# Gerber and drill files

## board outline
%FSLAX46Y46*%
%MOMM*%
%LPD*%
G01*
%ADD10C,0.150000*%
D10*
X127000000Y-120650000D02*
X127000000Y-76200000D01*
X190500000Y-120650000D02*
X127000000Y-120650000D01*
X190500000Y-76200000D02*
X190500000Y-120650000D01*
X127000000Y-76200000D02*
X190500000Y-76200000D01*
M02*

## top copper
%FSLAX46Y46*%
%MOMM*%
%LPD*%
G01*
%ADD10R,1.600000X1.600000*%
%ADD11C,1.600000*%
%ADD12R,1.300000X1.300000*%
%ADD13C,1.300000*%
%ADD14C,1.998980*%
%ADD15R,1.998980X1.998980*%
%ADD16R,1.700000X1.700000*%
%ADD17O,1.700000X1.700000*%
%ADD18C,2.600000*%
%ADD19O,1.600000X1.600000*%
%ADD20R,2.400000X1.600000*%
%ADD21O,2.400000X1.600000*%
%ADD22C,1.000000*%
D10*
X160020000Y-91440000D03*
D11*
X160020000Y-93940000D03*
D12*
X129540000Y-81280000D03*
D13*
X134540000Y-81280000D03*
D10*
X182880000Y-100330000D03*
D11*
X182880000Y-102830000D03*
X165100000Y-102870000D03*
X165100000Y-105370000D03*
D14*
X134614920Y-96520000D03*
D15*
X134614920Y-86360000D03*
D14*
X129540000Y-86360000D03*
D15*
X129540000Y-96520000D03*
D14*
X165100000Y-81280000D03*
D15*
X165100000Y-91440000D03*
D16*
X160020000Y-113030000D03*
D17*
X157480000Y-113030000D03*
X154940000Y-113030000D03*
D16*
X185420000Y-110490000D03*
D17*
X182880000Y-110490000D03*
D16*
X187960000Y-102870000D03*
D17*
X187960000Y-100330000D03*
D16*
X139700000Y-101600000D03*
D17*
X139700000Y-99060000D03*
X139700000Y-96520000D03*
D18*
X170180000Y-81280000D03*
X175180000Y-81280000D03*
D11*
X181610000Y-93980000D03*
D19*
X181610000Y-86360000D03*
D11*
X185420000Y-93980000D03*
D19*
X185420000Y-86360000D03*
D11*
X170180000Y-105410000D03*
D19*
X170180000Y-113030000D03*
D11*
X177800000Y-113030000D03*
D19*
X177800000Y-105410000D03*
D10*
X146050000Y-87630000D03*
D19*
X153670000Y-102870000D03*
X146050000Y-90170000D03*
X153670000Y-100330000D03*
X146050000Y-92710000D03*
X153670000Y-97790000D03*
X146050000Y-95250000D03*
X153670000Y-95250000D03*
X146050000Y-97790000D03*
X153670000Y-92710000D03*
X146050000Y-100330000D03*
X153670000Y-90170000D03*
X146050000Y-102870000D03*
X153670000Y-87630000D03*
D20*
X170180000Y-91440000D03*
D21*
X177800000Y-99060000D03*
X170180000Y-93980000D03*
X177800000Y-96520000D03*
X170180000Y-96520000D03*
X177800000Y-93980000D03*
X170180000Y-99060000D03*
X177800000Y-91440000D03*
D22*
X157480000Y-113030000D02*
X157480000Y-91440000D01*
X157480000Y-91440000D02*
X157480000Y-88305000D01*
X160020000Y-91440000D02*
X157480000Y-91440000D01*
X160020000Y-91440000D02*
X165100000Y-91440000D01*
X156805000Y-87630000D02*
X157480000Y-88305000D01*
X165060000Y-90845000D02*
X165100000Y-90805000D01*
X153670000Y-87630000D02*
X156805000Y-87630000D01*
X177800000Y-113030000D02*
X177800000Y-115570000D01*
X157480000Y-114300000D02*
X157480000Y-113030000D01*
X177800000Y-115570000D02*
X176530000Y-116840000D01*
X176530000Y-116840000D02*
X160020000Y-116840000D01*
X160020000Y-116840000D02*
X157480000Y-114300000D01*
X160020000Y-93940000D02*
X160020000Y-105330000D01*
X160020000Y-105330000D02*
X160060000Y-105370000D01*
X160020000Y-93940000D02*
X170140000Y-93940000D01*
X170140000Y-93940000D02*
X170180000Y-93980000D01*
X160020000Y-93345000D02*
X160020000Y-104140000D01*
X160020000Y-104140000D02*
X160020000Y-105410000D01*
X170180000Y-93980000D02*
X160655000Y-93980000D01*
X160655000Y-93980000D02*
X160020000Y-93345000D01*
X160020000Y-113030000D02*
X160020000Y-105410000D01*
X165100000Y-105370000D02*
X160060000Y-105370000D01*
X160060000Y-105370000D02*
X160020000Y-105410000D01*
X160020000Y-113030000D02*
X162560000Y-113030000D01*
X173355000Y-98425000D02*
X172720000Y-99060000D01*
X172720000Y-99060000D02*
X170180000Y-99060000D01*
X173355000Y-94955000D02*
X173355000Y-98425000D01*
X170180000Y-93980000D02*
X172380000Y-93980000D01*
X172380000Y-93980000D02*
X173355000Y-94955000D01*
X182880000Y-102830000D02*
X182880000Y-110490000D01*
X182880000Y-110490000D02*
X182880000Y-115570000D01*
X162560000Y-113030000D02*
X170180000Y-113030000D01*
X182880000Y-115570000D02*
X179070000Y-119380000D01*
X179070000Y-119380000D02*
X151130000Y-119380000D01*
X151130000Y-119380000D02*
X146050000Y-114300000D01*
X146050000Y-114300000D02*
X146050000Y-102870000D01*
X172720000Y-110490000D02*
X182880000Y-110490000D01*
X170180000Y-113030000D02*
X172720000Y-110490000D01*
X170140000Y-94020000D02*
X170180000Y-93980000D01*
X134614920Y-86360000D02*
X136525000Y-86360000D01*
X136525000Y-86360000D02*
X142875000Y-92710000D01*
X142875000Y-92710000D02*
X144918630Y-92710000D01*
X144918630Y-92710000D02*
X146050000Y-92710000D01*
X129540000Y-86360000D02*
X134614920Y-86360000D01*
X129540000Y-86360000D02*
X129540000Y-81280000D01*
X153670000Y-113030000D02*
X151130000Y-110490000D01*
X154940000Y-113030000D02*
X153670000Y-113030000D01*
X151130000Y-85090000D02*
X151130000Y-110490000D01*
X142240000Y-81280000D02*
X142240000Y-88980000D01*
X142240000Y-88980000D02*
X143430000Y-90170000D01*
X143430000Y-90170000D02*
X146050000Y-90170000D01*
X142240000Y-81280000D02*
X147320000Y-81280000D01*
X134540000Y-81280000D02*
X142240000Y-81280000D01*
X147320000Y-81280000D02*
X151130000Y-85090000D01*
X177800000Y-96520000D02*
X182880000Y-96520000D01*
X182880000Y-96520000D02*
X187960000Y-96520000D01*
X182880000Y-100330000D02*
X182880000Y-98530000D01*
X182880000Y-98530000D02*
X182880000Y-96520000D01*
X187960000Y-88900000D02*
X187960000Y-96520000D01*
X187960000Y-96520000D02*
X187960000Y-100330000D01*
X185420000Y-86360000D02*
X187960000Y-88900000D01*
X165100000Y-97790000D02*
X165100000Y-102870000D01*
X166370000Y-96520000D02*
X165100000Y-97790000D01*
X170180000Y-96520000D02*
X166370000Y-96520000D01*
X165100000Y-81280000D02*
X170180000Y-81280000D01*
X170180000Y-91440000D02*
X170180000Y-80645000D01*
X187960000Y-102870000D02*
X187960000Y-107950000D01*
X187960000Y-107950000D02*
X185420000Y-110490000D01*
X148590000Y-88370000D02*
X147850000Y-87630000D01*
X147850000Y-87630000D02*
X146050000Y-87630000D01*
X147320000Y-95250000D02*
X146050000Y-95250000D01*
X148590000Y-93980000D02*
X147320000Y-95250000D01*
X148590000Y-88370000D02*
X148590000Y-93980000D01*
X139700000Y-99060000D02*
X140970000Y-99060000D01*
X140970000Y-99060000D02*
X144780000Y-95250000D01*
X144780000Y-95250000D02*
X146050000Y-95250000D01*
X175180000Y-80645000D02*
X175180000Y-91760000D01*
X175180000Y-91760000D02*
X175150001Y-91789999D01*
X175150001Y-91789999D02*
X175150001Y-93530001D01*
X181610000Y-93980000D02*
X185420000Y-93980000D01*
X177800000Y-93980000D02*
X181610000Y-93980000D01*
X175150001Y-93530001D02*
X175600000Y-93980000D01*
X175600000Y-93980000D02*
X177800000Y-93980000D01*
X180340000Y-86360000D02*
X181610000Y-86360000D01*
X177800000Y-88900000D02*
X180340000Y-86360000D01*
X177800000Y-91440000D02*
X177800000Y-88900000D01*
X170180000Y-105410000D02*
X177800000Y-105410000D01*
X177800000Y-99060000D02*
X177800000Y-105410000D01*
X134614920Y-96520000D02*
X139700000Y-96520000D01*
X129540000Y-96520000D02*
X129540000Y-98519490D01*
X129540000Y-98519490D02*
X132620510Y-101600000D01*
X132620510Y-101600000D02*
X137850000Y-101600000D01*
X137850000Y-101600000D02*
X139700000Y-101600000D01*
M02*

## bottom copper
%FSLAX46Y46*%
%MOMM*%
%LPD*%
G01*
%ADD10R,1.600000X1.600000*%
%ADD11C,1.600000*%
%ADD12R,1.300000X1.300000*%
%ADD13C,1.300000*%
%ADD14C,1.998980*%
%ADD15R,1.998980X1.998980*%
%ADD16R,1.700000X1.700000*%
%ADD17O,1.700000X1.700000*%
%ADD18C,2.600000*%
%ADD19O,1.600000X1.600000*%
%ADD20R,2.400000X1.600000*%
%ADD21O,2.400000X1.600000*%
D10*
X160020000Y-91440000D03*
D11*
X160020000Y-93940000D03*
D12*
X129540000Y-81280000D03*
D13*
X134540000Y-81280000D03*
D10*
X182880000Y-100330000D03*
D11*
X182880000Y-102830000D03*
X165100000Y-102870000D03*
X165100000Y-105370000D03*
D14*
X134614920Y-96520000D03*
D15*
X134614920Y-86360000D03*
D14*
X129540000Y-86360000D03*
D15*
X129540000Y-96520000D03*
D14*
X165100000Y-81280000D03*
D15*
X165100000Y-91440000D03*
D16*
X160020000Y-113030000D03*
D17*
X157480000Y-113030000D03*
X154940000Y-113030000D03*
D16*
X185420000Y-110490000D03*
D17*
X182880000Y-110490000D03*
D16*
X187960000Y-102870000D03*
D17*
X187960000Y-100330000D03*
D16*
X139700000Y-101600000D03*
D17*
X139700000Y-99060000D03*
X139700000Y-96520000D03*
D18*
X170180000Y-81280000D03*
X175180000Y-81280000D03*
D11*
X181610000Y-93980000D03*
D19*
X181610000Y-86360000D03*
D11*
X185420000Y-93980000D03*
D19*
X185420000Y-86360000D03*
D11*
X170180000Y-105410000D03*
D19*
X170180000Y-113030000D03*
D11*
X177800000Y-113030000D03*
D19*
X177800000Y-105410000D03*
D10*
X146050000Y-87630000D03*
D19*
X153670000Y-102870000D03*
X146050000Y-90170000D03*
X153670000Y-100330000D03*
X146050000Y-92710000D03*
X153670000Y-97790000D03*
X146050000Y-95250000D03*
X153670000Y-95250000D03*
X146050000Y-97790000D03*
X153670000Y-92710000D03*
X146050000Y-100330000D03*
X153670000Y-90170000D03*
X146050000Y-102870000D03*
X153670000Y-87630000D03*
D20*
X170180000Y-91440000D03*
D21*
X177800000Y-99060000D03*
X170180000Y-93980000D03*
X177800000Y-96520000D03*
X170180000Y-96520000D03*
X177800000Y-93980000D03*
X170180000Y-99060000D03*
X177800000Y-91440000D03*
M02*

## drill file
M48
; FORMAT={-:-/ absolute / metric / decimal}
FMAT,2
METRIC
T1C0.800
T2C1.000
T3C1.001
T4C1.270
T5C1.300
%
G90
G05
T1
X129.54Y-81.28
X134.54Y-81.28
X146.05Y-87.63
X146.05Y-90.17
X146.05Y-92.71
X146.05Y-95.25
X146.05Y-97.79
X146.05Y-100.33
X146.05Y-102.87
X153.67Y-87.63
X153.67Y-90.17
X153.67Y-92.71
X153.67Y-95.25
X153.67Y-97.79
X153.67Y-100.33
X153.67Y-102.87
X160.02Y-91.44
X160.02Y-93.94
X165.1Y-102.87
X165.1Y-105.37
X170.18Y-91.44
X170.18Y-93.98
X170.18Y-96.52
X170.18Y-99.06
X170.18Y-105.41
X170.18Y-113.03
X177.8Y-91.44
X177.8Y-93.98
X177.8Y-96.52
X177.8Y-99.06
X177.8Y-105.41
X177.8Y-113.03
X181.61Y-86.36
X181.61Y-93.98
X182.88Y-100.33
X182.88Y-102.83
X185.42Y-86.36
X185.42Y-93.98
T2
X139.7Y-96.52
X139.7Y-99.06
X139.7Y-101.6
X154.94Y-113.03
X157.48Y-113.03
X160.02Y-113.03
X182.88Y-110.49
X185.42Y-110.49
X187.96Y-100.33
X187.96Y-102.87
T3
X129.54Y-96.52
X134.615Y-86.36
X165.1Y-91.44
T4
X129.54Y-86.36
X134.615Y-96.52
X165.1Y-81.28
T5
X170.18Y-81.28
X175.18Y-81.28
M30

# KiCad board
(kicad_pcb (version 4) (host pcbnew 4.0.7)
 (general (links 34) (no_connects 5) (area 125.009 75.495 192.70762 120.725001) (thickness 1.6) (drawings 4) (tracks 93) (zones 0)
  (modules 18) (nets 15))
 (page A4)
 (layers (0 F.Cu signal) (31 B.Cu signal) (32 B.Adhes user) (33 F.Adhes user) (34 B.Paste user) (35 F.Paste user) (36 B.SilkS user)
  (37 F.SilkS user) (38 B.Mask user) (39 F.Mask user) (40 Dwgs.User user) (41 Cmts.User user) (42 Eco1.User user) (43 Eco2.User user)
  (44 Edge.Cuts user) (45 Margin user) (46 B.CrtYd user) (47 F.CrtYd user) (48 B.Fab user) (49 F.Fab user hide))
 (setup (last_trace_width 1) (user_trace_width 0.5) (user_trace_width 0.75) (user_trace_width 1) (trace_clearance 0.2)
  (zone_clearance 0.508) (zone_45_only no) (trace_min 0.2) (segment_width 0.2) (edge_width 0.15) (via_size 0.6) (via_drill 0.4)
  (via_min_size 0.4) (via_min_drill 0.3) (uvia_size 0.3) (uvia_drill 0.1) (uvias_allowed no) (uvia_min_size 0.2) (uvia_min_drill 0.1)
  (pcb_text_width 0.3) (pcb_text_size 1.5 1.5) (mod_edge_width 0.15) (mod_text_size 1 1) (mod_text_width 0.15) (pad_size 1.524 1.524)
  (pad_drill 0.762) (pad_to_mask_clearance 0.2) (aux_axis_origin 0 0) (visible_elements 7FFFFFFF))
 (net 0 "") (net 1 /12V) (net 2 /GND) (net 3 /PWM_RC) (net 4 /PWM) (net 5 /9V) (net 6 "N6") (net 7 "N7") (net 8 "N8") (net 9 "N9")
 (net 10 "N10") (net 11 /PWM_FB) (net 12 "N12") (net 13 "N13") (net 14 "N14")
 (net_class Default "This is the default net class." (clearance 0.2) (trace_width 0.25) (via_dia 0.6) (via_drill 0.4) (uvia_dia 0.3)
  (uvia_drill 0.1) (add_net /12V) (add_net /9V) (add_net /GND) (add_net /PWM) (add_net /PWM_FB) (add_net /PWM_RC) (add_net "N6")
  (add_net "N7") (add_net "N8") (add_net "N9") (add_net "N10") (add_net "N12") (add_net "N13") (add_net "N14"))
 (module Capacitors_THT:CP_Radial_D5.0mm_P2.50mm (layer F.Cu) (at 160.02 91.44 270)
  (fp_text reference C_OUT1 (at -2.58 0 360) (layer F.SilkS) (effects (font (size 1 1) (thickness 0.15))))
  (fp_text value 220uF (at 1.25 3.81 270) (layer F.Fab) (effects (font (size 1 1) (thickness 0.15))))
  (pad 1 thru_hole rect (at 0 0 270) (size 1.6 1.6) (drill 0.8) (layers *.Cu *.Mask) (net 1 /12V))
  (pad 2 thru_hole circle (at 2.5 0 270) (size 1.6 1.6) (drill 0.8) (layers *.Cu *.Mask) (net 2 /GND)))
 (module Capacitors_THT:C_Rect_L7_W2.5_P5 (layer F.Cu) (at 129.54 81.28)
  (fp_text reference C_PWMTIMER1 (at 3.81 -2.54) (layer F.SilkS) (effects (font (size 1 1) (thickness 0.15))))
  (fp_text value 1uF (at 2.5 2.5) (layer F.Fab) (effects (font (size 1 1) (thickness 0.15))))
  (pad 1 thru_hole rect (at 0 0) (size 1.3 1.3) (drill 0.8) (layers *.Cu *.Mask) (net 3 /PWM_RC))
  (pad 2 thru_hole circle (at 5 0) (size 1.3 1.3) (drill 0.8) (layers *.Cu *.Mask) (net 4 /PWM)))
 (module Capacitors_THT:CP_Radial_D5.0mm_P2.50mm (layer F.Cu) (at 182.88 100.33 270)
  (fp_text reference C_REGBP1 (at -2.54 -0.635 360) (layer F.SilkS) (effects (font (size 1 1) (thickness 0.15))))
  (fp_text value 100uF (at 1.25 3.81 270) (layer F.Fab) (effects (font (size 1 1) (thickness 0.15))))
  (pad 1 thru_hole rect (at 0 0 270) (size 1.6 1.6) (drill 0.8) (layers *.Cu *.Mask) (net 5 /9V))
  (pad 2 thru_hole circle (at 2.5 0 270) (size 1.6 1.6) (drill 0.8) (layers *.Cu *.Mask) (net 2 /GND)))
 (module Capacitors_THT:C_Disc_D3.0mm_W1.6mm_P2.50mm (layer F.Cu) (at 165.1 102.87 270)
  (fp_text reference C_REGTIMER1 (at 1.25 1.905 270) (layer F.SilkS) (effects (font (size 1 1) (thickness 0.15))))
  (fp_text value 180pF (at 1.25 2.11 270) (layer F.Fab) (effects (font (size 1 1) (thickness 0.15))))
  (pad 1 thru_hole circle (at 0 0 270) (size 1.6 1.6) (drill 0.8) (layers *.Cu *.Mask) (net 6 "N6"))
  (pad 2 thru_hole circle (at 2.5 0 270) (size 1.6 1.6) (drill 0.8) (layers *.Cu *.Mask) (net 2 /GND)))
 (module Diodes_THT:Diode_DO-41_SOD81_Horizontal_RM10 (layer F.Cu) (at 134.61238 86.36 270)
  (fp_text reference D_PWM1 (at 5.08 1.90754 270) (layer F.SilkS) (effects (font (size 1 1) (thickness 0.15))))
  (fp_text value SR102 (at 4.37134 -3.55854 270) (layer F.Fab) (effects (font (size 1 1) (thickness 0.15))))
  (pad 2 thru_hole circle (at 10.16 -0.00254 90) (size 1.99898 1.99898) (drill 1.27) (layers *.Cu *.Mask) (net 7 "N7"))
  (pad 1 thru_hole rect (at 0 -0.00254 90) (size 1.99898 1.99898) (drill 1.00076) (layers *.Cu *.Mask) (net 3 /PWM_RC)))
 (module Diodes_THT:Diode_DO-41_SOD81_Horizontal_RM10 (layer F.Cu) (at 129.54254 96.52 90)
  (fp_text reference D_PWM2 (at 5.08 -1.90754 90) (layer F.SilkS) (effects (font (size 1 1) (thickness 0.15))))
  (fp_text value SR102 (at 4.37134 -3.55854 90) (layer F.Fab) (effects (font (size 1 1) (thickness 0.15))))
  (pad 2 thru_hole circle (at 10.16 -0.00254 270) (size 1.99898 1.99898) (drill 1.27) (layers *.Cu *.Mask) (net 3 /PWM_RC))
  (pad 1 thru_hole rect (at 0 -0.00254 270) (size 1.99898 1.99898) (drill 1.00076) (layers *.Cu *.Mask) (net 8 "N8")))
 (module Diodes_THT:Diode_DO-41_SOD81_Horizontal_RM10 (layer F.Cu) (at 165.10254 91.44 90)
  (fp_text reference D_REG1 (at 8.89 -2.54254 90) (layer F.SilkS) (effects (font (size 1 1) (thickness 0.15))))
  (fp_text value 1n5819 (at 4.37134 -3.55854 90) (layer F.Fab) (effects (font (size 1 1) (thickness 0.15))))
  (pad 2 thru_hole circle (at 10.16 -0.00254 270) (size 1.99898 1.99898) (drill 1.27) (layers *.Cu *.Mask) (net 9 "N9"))
  (pad 1 thru_hole rect (at 0 -0.00254 270) (size 1.99898 1.99898) (drill 1.00076) (layers *.Cu *.Mask) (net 1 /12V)))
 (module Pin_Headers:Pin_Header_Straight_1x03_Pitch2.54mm (layer F.Cu) (at 160.02 113.03 270)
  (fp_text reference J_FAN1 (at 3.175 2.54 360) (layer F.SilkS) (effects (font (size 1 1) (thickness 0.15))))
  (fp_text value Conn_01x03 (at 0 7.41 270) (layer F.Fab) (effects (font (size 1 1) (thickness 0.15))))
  (pad 1 thru_hole rect (at 0 0 270) (size 1.7 1.7) (drill 1) (layers *.Cu *.Mask) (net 2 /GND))
  (pad 2 thru_hole oval (at 0 2.54 270) (size 1.7 1.7) (drill 1) (layers *.Cu *.Mask) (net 1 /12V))
  (pad 3 thru_hole oval (at 0 5.08 270) (size 1.7 1.7) (drill 1) (layers *.Cu *.Mask) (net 4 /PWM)))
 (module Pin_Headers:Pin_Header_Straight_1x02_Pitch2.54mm (layer F.Cu) (at 185.42 110.49 270)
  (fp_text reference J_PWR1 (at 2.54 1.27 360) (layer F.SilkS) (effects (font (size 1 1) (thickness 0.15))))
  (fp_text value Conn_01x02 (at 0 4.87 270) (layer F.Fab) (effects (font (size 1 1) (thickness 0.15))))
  (pad 1 thru_hole rect (at 0 0 270) (size 1.7 1.7) (drill 1) (layers *.Cu *.Mask) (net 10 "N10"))
  (pad 2 thru_hole oval (at 0 2.54 270) (size 1.7 1.7) (drill 1) (layers *.Cu *.Mask) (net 2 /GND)))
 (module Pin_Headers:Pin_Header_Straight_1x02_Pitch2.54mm (layer F.Cu) (at 187.96 102.87 180)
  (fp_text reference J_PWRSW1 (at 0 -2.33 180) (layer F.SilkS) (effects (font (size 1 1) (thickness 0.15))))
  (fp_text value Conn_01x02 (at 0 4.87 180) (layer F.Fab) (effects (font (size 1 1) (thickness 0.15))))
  (pad 1 thru_hole rect (at 0 0 180) (size 1.7 1.7) (drill 1) (layers *.Cu *.Mask) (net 10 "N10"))
  (pad 2 thru_hole oval (at 0 2.54 180) (size 1.7 1.7) (drill 1) (layers *.Cu *.Mask) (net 5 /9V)))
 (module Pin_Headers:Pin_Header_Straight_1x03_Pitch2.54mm (layer F.Cu) (at 139.7 101.6 180)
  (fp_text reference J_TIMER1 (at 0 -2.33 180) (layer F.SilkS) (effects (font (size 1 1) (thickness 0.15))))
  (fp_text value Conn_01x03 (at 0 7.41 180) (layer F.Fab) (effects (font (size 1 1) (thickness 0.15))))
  (pad 1 thru_hole rect (at 0 0 180) (size 1.7 1.7) (drill 1) (layers *.Cu *.Mask) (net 8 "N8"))
  (pad 2 thru_hole oval (at 0 2.54 180) (size 1.7 1.7) (drill 1) (layers *.Cu *.Mask) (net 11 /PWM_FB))
  (pad 3 thru_hole oval (at 0 5.08 180) (size 1.7 1.7) (drill 1) (layers *.Cu *.Mask) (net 7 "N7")))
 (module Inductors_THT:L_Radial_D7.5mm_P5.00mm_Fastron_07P (layer F.Cu) (at 170.18 81.28)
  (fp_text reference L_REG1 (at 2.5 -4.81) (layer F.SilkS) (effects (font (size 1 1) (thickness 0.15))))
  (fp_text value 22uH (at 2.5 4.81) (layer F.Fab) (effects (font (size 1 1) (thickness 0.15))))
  (pad 1 thru_hole circle (at 0 0) (size 2.6 2.6) (drill 1.3) (layers *.Cu *.Mask) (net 9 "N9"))
  (pad 2 thru_hole circle (at 5 0) (size 2.6 2.6) (drill 1.3) (layers *.Cu *.Mask) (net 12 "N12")))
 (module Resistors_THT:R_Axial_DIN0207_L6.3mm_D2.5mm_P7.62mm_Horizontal (layer F.Cu) (at 181.61 93.98 90)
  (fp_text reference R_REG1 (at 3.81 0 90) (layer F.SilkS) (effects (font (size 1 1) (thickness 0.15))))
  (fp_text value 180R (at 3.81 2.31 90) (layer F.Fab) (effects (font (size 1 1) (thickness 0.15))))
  (pad 1 thru_hole circle (at 0 0 90) (size 1.6 1.6) (drill 0.8) (layers *.Cu *.Mask) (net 12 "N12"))
  (pad 2 thru_hole oval (at 7.62 0 90) (size 1.6 1.6) (drill 0.8) (layers *.Cu *.Mask) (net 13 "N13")))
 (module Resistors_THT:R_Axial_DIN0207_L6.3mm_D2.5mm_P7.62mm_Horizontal (layer F.Cu) (at 185.42 93.98 90)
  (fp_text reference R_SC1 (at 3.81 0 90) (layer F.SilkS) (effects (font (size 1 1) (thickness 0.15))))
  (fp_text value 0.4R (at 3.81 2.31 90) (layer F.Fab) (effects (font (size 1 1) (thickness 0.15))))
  (pad 1 thru_hole circle (at 0 0 90) (size 1.6 1.6) (drill 0.8) (layers *.Cu *.Mask) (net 12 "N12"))
  (pad 2 thru_hole oval (at 7.62 0 90) (size 1.6 1.6) (drill 0.8) (layers *.Cu *.Mask) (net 5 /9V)))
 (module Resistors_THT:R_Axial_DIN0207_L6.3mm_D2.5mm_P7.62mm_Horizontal (layer F.Cu) (at 170.18 105.41 270)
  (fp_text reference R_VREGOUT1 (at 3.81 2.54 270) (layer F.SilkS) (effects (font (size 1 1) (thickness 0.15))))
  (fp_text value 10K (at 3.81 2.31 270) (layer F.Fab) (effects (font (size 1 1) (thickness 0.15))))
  (pad 1 thru_hole circle (at 0 0 270) (size 1.6 1.6) (drill 0.8) (layers *.Cu *.Mask) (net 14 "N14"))
  (pad 2 thru_hole oval (at 7.62 0 270) (size 1.6 1.6) (drill 0.8) (layers *.Cu *.Mask) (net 2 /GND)))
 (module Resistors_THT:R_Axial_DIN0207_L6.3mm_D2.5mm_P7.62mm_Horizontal (layer F.Cu) (at 177.8 113.03 90)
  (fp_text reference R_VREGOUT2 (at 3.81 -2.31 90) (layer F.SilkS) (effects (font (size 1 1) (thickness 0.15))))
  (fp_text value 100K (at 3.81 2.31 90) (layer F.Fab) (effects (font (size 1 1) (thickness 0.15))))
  (pad 1 thru_hole circle (at 0 0 90) (size 1.6 1.6) (drill 0.8) (layers *.Cu *.Mask) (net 1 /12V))
  (pad 2 thru_hole oval (at 7.62 0 90) (size 1.6 1.6) (drill 0.8) (layers *.Cu *.Mask) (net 14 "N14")))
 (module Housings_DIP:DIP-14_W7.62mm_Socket (layer F.Cu) (at 146.05 87.63)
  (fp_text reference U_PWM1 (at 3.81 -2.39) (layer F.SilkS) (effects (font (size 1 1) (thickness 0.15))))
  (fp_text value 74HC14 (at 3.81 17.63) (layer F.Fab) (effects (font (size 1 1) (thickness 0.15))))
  (pad 1 thru_hole rect (at 0 0) (size 1.6 1.6) (drill 0.8) (layers *.Cu *.Mask) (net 11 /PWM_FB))
  (pad 8 thru_hole oval (at 7.62 15.24) (size 1.6 1.6) (drill 0.8) (layers *.Cu *.Mask))
  (pad 2 thru_hole oval (at 0 2.54) (size 1.6 1.6) (drill 0.8) (layers *.Cu *.Mask) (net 4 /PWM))
  (pad 9 thru_hole oval (at 7.62 12.7) (size 1.6 1.6) (drill 0.8) (layers *.Cu *.Mask))
  (pad 3 thru_hole oval (at 0 5.08) (size 1.6 1.6) (drill 0.8) (layers *.Cu *.Mask) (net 3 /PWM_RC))
  (pad 10 thru_hole oval (at 7.62 10.16) (size 1.6 1.6) (drill 0.8) (layers *.Cu *.Mask))
  (pad 4 thru_hole oval (at 0 7.62) (size 1.6 1.6) (drill 0.8) (layers *.Cu *.Mask) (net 11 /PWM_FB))
  (pad 11 thru_hole oval (at 7.62 7.62) (size 1.6 1.6) (drill 0.8) (layers *.Cu *.Mask))
  (pad 5 thru_hole oval (at 0 10.16) (size 1.6 1.6) (drill 0.8) (layers *.Cu *.Mask))
  (pad 12 thru_hole oval (at 7.62 5.08) (size 1.6 1.6) (drill 0.8) (layers *.Cu *.Mask))
  (pad 6 thru_hole oval (at 0 12.7) (size 1.6 1.6) (drill 0.8) (layers *.Cu *.Mask))
  (pad 13 thru_hole oval (at 7.62 2.54) (size 1.6 1.6) (drill 0.8) (layers *.Cu *.Mask))
  (pad 7 thru_hole oval (at 0 15.24) (size 1.6 1.6) (drill 0.8) (layers *.Cu *.Mask) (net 2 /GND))
  (pad 14 thru_hole oval (at 7.62 0) (size 1.6 1.6) (drill 0.8) (layers *.Cu *.Mask) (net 1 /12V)))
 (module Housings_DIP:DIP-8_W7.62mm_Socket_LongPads (layer F.Cu) (at 170.18 91.44)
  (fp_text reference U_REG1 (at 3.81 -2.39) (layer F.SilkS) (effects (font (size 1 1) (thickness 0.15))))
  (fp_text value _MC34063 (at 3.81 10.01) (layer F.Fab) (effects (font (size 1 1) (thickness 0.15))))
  (pad 1 thru_hole rect (at 0 0) (size 2.4 1.6) (drill 0.8) (layers *.Cu *.Mask) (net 9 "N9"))
  (pad 5 thru_hole oval (at 7.62 7.62) (size 2.4 1.6) (drill 0.8) (layers *.Cu *.Mask) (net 14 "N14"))
  (pad 2 thru_hole oval (at 0 2.54) (size 2.4 1.6) (drill 0.8) (layers *.Cu *.Mask) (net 2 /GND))
  (pad 6 thru_hole oval (at 7.62 5.08) (size 2.4 1.6) (drill 0.8) (layers *.Cu *.Mask) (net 5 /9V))
  (pad 3 thru_hole oval (at 0 5.08) (size 2.4 1.6) (drill 0.8) (layers *.Cu *.Mask) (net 6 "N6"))
  (pad 7 thru_hole oval (at 7.62 2.54) (size 2.4 1.6) (drill 0.8) (layers *.Cu *.Mask) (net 12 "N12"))
  (pad 4 thru_hole oval (at 0 7.62) (size 2.4 1.6) (drill 0.8) (layers *.Cu *.Mask) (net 2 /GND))
  (pad 8 thru_hole oval (at 7.62 0) (size 2.4 1.6) (drill 0.8) (layers *.Cu *.Mask) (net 13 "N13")))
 (gr_line (start 127 120.65) (end 127 76.2) (layer Edge.Cuts) (width 0.15))
 (gr_line (start 190.5 120.65) (end 127 120.65) (layer Edge.Cuts) (width 0.15))
 (gr_line (start 190.5 76.2) (end 190.5 120.65) (layer Edge.Cuts) (width 0.15))
 (gr_line (start 127 76.2) (end 190.5 76.2) (layer Edge.Cuts) (width 0.15))
 (segment (start 157.48 113.03) (end 157.48 91.44) (width 1) (layer F.Cu) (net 1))
 (segment (start 157.48 91.44) (end 157.48 88.305) (width 1) (layer F.Cu) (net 1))
 (segment (start 160.02 91.44) (end 157.48 91.44) (width 1) (layer F.Cu) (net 1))
 (segment (start 160.02 91.44) (end 165.1 91.44) (width 1) (layer F.Cu) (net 1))
 (segment (start 156.805 87.63) (end 157.48 88.305) (width 1) (layer F.Cu) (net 1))
 (segment (start 165.06 90.845) (end 165.1 90.805) (width 1) (layer F.Cu) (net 1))
 (segment (start 153.67 87.63) (end 156.805 87.63) (width 1) (layer F.Cu) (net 1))
 (segment (start 177.8 113.03) (end 177.8 115.57) (width 1) (layer F.Cu) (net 1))
 (segment (start 157.48 114.3) (end 157.48 113.03) (width 1) (layer F.Cu) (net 1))
 (segment (start 177.8 115.57) (end 176.53 116.84) (width 1) (layer F.Cu) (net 1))
 (segment (start 176.53 116.84) (end 160.02 116.84) (width 1) (layer F.Cu) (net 1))
 (segment (start 160.02 116.84) (end 157.48 114.3) (width 1) (layer F.Cu) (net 1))
 (segment (start 160.02 93.94) (end 160.02 105.33) (width 1) (layer F.Cu) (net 2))
 (segment (start 160.02 105.33) (end 160.06 105.37) (width 1) (layer F.Cu) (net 2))
 (segment (start 160.02 93.94) (end 170.14 93.94) (width 1) (layer F.Cu) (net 2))
 (segment (start 170.14 93.94) (end 170.18 93.98) (width 1) (layer F.Cu) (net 2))
 (segment (start 160.02 93.345) (end 160.02 104.14) (width 1) (layer F.Cu) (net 2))
 (segment (start 160.02 104.14) (end 160.02 105.41) (width 1) (layer F.Cu) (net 2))
 (segment (start 170.18 93.98) (end 160.655 93.98) (width 1) (layer F.Cu) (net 2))
 (segment (start 160.655 93.98) (end 160.02 93.345) (width 1) (layer F.Cu) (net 2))
 (segment (start 160.02 113.03) (end 160.02 105.41) (width 1) (layer F.Cu) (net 2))
 (segment (start 165.1 105.37) (end 160.06 105.37) (width 1) (layer F.Cu) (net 2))
 (segment (start 160.06 105.37) (end 160.02 105.41) (width 1) (layer F.Cu) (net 2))
 (segment (start 160.02 113.03) (end 162.56 113.03) (width 1) (layer F.Cu) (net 2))
 (segment (start 173.355 98.425) (end 172.72 99.06) (width 1) (layer F.Cu) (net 2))
 (segment (start 172.72 99.06) (end 170.18 99.06) (width 1) (layer F.Cu) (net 2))
 (segment (start 173.355 94.955) (end 173.355 98.425) (width 1) (layer F.Cu) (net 2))
 (segment (start 170.18 93.98) (end 172.38 93.98) (width 1) (layer F.Cu) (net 2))
 (segment (start 172.38 93.98) (end 173.355 94.955) (width 1) (layer F.Cu) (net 2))
 (segment (start 182.88 102.83) (end 182.88 110.49) (width 1) (layer F.Cu) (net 2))
 (segment (start 182.88 110.49) (end 182.88 115.57) (width 1) (layer F.Cu) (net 2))
 (segment (start 162.56 113.03) (end 170.18 113.03) (width 1) (layer F.Cu) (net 2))
 (segment (start 182.88 115.57) (end 179.07 119.38) (width 1) (layer F.Cu) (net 2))
 (segment (start 179.07 119.38) (end 151.13 119.38) (width 1) (layer F.Cu) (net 2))
 (segment (start 151.13 119.38) (end 146.05 114.3) (width 1) (layer F.Cu) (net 2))
 (segment (start 146.05 114.3) (end 146.05 102.87) (width 1) (layer F.Cu) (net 2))
 (segment (start 172.72 110.49) (end 182.88 110.49) (width 1) (layer F.Cu) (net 2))
 (segment (start 170.18 113.03) (end 172.72 110.49) (width 1) (layer F.Cu) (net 2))
 (segment (start 170.14 94.02) (end 170.18 93.98) (width 1) (layer F.Cu) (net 2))
 (segment (start 134.61492 86.36) (end 136.525 86.36) (width 1) (layer F.Cu) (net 3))
 (segment (start 136.525 86.36) (end 142.875 92.71) (width 1) (layer F.Cu) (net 3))
 (segment (start 142.875 92.71) (end 144.91863 92.71) (width 1) (layer F.Cu) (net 3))
 (segment (start 144.91863 92.71) (end 146.05 92.71) (width 1) (layer F.Cu) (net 3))
 (segment (start 129.54 86.36) (end 134.61492 86.36) (width 1) (layer F.Cu) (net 3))
 (segment (start 129.54 86.36) (end 129.54 81.28) (width 1) (layer F.Cu) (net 3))
 (segment (start 153.67 113.03) (end 151.13 110.49) (width 1) (layer F.Cu) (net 4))
 (segment (start 154.94 113.03) (end 153.67 113.03) (width 1) (layer F.Cu) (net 4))
 (segment (start 151.13 85.09) (end 151.13 110.49) (width 1) (layer F.Cu) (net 4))
 (segment (start 142.24 81.28) (end 142.24 88.98) (width 1) (layer F.Cu) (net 4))
 (segment (start 142.24 88.98) (end 143.43 90.17) (width 1) (layer F.Cu) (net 4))
 (segment (start 143.43 90.17) (end 146.05 90.17) (width 1) (layer F.Cu) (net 4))
 (segment (start 142.24 81.28) (end 147.32 81.28) (width 1) (layer F.Cu) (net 4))
 (segment (start 134.54 81.28) (end 142.24 81.28) (width 1) (layer F.Cu) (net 4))
 (segment (start 147.32 81.28) (end 151.13 85.09) (width 1) (layer F.Cu) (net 4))
 (segment (start 177.8 96.52) (end 182.88 96.52) (width 1) (layer F.Cu) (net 5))
 (segment (start 182.88 96.52) (end 187.96 96.52) (width 1) (layer F.Cu) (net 5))
 (segment (start 182.88 100.33) (end 182.88 98.53) (width 1) (layer F.Cu) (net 5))
 (segment (start 182.88 98.53) (end 182.88 96.52) (width 1) (layer F.Cu) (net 5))
 (segment (start 187.96 88.9) (end 187.96 96.52) (width 1) (layer F.Cu) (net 5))
 (segment (start 187.96 96.52) (end 187.96 100.33) (width 1) (layer F.Cu) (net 5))
 (segment (start 185.42 86.36) (end 187.96 88.9) (width 1) (layer F.Cu) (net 5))
 (segment (start 165.1 97.79) (end 165.1 102.87) (width 1) (layer F.Cu) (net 6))
 (segment (start 166.37 96.52) (end 165.1 97.79) (width 1) (layer F.Cu) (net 6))
 (segment (start 170.18 96.52) (end 166.37 96.52) (width 1) (layer F.Cu) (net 6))
 (segment (start 165.1 81.28) (end 170.18 81.28) (width 1) (layer F.Cu) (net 9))
 (segment (start 170.18 91.44) (end 170.18 80.645) (width 1) (layer F.Cu) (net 9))
 (segment (start 187.96 102.87) (end 187.96 107.95) (width 1) (layer F.Cu) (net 10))
 (segment (start 187.96 107.95) (end 185.42 110.49) (width 1) (layer F.Cu) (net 10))
 (segment (start 148.59 88.37) (end 147.85 87.63) (width 1) (layer F.Cu) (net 11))
 (segment (start 147.85 87.63) (end 146.05 87.63) (width 1) (layer F.Cu) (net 11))
 (segment (start 147.32 95.25) (end 146.05 95.25) (width 1) (layer F.Cu) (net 11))
 (segment (start 148.59 93.98) (end 147.32 95.25) (width 1) (layer F.Cu) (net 11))
 (segment (start 148.59 88.37) (end 148.59 93.98) (width 1) (layer F.Cu) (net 11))
 (segment (start 139.7 99.06) (end 140.97 99.06) (width 1) (layer F.Cu) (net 11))
 (segment (start 140.97 99.06) (end 144.78 95.25) (width 1) (layer F.Cu) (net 11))
 (segment (start 144.78 95.25) (end 146.05 95.25) (width 1) (layer F.Cu) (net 11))
 (segment (start 175.18 80.645) (end 175.18 91.76) (width 1) (layer F.Cu) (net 12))
 (segment (start 175.18 91.76) (end 175.150001 91.789999) (width 1) (layer F.Cu) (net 12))
 (segment (start 175.150001 91.789999) (end 175.150001 93.530001) (width 1) (layer F.Cu) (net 12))
 (segment (start 181.61 93.98) (end 185.42 93.98) (width 1) (layer F.Cu) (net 12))
 (segment (start 177.8 93.98) (end 181.61 93.98) (width 1) (layer F.Cu) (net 12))
 (segment (start 175.150001 93.530001) (end 175.6 93.98) (width 1) (layer F.Cu) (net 12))
 (segment (start 175.6 93.98) (end 177.8 93.98) (width 1) (layer F.Cu) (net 12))
 (segment (start 180.34 86.36) (end 181.61 86.36) (width 1) (layer F.Cu) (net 13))
 (segment (start 177.8 88.9) (end 180.34 86.36) (width 1) (layer F.Cu) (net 13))
 (segment (start 177.8 91.44) (end 177.8 88.9) (width 1) (layer F.Cu) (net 13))
 (segment (start 170.18 105.41) (end 177.8 105.41) (width 1) (layer F.Cu) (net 14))
 (segment (start 177.8 99.06) (end 177.8 105.41) (width 1) (layer F.Cu) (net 14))
 (segment (start 134.61492 96.52) (end 139.7 96.52) (width 1) (layer F.Cu) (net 7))
 (segment (start 129.54 96.52) (end 129.54 98.51949) (width 1) (layer F.Cu) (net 8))
 (segment (start 129.54 98.51949) (end 132.62051 101.6) (width 1) (layer F.Cu) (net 8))
 (segment (start 132.62051 101.6) (end 137.85 101.6) (width 1) (layer F.Cu) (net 8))
 (segment (start 137.85 101.6) (end 139.7 101.6) (width 1) (layer F.Cu) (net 8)))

